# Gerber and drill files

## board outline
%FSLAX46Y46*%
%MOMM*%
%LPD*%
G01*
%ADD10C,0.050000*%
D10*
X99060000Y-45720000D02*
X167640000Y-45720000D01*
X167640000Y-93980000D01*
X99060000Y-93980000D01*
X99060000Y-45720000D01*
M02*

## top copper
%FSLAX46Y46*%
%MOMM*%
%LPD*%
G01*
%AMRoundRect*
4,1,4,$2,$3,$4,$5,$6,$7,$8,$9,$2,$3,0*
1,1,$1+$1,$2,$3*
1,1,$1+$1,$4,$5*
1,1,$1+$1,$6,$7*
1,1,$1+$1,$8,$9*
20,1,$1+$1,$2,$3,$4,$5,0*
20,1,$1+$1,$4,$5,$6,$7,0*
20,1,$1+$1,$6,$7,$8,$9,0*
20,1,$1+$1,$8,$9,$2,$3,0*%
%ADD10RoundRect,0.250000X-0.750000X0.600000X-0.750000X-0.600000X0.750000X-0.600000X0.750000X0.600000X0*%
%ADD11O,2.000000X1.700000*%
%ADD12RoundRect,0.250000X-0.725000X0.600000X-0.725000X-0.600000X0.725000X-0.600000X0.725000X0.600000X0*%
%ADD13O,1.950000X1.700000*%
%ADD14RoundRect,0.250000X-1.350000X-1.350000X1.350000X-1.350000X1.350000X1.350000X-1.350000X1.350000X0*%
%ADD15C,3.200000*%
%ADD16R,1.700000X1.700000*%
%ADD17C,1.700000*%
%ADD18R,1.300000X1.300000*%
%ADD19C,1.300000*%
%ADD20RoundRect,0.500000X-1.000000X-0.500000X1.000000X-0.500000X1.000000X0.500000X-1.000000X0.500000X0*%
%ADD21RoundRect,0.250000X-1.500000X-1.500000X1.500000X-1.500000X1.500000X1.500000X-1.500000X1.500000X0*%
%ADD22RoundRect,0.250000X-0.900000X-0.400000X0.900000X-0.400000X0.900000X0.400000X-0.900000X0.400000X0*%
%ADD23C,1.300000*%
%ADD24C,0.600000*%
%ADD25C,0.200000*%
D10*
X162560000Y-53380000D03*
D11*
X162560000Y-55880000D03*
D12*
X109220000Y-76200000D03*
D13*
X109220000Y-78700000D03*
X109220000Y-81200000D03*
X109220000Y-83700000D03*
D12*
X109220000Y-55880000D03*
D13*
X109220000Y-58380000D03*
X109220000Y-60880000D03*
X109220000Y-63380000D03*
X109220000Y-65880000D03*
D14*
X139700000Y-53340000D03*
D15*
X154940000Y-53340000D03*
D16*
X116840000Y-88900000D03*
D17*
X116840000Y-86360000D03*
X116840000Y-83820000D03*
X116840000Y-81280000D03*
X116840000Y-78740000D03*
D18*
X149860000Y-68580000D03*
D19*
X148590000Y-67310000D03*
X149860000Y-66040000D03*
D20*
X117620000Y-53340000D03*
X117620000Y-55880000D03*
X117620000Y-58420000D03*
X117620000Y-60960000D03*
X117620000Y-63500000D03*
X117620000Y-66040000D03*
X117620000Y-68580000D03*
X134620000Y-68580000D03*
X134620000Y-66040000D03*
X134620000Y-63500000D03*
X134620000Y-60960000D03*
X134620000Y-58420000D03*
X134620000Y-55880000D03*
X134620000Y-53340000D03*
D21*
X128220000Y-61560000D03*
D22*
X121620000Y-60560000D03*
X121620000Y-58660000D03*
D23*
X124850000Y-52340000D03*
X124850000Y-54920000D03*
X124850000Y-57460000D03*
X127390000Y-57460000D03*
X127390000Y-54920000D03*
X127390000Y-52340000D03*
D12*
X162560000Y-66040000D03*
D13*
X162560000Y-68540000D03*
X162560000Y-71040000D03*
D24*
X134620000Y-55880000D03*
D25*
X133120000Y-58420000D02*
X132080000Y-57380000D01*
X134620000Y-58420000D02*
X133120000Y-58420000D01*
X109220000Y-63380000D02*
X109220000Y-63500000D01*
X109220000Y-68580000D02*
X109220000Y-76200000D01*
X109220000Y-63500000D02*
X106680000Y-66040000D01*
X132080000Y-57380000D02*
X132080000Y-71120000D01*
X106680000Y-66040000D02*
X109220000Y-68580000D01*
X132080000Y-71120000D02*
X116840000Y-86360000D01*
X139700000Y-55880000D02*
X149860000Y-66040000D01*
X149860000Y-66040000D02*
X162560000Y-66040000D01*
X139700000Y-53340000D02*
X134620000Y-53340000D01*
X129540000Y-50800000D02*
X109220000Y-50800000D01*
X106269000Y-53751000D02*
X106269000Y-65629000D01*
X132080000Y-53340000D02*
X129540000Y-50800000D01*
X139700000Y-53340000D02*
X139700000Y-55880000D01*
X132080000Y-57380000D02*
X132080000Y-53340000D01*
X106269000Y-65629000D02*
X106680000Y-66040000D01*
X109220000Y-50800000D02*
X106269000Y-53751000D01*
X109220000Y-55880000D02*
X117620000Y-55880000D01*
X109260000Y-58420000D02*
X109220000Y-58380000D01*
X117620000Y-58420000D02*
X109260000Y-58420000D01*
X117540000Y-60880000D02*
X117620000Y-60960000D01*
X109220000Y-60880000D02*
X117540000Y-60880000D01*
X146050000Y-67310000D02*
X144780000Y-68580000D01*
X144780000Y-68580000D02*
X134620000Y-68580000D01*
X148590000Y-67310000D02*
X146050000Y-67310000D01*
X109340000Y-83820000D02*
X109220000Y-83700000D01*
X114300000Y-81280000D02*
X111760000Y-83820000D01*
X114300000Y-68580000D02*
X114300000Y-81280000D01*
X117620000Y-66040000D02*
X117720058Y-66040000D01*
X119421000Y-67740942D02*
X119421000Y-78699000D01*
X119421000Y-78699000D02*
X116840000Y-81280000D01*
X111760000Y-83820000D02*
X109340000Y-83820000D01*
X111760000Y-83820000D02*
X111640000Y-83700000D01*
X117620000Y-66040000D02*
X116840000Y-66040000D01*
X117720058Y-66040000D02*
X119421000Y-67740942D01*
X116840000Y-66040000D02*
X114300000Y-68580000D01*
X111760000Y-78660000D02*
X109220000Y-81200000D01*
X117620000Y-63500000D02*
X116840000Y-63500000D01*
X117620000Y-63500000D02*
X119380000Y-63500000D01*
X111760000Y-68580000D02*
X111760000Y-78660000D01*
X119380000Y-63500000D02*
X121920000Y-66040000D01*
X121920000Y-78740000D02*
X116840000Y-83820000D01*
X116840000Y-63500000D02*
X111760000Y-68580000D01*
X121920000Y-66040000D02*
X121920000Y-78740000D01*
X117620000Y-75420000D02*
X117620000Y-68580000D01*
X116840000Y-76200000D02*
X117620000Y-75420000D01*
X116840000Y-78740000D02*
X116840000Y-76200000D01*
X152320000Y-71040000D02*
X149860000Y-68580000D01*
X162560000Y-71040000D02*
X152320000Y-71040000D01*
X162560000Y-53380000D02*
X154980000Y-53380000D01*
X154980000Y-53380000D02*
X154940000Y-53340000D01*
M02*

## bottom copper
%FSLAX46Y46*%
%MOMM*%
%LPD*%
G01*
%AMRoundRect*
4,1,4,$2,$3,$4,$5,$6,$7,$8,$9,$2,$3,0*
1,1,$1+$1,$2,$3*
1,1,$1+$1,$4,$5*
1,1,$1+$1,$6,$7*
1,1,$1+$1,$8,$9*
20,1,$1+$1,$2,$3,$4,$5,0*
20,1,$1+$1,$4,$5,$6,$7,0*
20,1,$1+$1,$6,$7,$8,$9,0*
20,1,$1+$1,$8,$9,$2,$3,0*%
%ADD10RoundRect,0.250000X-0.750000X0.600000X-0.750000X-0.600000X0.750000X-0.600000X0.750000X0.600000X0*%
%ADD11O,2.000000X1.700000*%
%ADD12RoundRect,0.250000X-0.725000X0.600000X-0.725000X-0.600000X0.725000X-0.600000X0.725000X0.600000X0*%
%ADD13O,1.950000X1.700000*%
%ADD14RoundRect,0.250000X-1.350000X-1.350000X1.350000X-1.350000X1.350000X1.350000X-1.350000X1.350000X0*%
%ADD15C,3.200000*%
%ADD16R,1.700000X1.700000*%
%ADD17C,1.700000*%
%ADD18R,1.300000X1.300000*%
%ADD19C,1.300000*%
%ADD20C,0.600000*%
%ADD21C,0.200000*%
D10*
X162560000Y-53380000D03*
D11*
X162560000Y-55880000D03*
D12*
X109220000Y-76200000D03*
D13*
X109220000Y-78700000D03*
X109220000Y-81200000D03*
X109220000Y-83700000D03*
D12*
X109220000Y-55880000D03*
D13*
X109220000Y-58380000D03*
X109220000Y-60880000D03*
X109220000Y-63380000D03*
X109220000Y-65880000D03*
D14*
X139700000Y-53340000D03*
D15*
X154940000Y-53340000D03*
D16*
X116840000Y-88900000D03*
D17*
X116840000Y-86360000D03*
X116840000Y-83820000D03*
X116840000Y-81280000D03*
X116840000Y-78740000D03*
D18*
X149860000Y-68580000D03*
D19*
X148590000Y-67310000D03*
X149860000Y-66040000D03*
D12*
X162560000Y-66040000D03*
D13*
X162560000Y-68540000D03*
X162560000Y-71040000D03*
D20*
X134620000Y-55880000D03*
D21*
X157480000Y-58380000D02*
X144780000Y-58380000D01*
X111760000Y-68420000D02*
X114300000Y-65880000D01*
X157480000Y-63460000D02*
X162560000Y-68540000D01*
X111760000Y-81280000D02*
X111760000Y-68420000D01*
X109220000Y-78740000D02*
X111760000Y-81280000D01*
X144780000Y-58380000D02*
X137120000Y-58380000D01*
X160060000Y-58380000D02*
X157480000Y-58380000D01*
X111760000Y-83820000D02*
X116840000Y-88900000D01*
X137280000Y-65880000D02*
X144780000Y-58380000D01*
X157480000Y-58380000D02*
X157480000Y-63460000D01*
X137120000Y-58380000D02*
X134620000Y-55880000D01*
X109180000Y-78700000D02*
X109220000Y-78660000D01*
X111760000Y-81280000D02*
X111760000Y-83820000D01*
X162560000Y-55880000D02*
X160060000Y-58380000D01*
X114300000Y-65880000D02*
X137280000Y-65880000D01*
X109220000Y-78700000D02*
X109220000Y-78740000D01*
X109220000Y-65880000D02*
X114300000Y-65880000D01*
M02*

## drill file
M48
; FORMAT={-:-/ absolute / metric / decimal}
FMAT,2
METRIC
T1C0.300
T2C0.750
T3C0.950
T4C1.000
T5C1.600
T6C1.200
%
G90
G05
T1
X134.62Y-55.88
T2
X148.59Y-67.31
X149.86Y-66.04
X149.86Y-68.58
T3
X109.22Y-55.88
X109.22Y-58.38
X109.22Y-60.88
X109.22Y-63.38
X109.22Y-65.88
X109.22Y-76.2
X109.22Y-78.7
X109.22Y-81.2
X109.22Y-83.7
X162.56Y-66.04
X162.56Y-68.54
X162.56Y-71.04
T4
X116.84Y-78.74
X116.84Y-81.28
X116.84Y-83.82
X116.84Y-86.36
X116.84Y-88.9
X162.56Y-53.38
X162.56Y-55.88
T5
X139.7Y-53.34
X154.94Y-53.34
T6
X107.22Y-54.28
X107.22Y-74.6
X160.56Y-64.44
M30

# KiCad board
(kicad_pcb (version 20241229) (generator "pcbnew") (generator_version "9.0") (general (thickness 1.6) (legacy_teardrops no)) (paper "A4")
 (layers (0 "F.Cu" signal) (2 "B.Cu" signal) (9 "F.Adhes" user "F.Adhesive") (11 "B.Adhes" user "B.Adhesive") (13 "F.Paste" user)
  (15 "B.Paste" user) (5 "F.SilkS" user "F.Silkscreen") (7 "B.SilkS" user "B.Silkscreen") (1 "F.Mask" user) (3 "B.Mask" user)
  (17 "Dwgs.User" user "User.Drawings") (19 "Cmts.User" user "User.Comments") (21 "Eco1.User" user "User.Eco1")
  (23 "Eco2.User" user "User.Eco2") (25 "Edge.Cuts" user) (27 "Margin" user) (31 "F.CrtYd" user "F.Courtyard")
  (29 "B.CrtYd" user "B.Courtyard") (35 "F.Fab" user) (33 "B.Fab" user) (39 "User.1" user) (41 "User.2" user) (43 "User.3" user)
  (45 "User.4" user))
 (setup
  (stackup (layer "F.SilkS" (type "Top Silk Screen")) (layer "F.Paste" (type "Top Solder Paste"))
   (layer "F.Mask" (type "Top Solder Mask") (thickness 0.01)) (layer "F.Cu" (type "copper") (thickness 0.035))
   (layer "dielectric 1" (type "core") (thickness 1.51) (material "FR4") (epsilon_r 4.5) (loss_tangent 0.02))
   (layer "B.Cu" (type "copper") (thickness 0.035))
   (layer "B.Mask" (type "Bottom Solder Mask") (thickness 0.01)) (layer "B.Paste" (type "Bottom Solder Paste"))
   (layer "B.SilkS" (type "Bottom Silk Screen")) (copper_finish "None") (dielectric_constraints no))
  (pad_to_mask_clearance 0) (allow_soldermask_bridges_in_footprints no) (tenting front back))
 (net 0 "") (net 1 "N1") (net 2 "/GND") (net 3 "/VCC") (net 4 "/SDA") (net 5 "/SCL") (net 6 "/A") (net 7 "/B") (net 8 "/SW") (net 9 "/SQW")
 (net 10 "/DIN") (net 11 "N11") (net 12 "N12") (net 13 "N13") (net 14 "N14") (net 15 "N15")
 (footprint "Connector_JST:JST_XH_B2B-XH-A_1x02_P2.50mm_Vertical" (layer "F.Cu") (at 162.56 53.38 -90)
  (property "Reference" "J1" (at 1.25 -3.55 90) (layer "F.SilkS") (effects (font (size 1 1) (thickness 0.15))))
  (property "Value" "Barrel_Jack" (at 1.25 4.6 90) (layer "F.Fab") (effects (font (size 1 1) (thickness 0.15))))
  (pad "1" thru_hole roundrect (at 0 0 270) (size 1.7 2) (drill 1) (layers "*.Cu" "*.Mask") (remove_unused_layers no)
   (roundrect_rratio 0.147059) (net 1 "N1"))
  (pad "2" thru_hole oval (at 2.5 0 270) (size 1.7 2) (drill 1) (layers "*.Cu" "*.Mask") (remove_unused_layers no) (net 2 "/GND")))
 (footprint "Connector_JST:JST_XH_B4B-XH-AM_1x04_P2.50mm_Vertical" (layer "F.Cu") (at 109.22 76.2 -90)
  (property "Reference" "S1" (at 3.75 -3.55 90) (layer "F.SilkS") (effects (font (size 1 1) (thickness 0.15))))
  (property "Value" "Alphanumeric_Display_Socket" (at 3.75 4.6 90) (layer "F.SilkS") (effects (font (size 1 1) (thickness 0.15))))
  (pad "" np_thru_hole circle (at -1.6 2 270) (size 1.2 1.2) (drill 1.2) (layers "*.Cu" "*.Mask"))
  (pad "1" thru_hole roundrect (at 0 0 270) (size 1.7 1.95) (drill 0.95) (layers "*.Cu" "*.Mask") (remove_unused_layers no)
   (roundrect_rratio 0.147059) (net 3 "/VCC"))
  (pad "2" thru_hole oval (at 2.5 0 270) (size 1.7 1.95) (drill 0.95) (layers "*.Cu" "*.Mask") (remove_unused_layers no) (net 2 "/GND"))
  (pad "3" thru_hole oval (at 5 0 270) (size 1.7 1.95) (drill 0.95) (layers "*.Cu" "*.Mask") (remove_unused_layers no) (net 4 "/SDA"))
  (pad "4" thru_hole oval (at 7.5 0 270) (size 1.7 1.95) (drill 0.95) (layers "*.Cu" "*.Mask") (remove_unused_layers no) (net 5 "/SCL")))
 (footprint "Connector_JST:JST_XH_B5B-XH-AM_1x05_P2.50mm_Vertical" (layer "F.Cu") (at 109.22 55.88 -90)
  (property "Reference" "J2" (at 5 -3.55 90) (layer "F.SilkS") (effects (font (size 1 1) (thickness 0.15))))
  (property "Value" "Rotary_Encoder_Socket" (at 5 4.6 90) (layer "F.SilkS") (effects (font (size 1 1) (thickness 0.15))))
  (pad "" np_thru_hole circle (at -1.6 2 270) (size 1.2 1.2) (drill 1.2) (layers "*.Cu" "*.Mask"))
  (pad "1" thru_hole roundrect (at 0 0 270) (size 1.7 1.95) (drill 0.95) (layers "*.Cu" "*.Mask") (remove_unused_layers no)
   (roundrect_rratio 0.147059) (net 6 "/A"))
  (pad "2" thru_hole oval (at 2.5 0 270) (size 1.7 1.95) (drill 0.95) (layers "*.Cu" "*.Mask") (remove_unused_layers no) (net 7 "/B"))
  (pad "3" thru_hole oval (at 5 0 270) (size 1.7 1.95) (drill 0.95) (layers "*.Cu" "*.Mask") (remove_unused_layers no) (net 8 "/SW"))
  (pad "4" thru_hole oval (at 7.5 0 270) (size 1.7 1.95) (drill 0.95) (layers "*.Cu" "*.Mask") (remove_unused_layers no) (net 3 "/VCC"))
  (pad "5" thru_hole oval (at 10 0 270) (size 1.7 1.95) (drill 0.95) (layers "*.Cu" "*.Mask") (remove_unused_layers no) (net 2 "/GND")))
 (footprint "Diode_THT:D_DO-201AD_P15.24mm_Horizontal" (layer "F.Cu") (at 139.7 53.34)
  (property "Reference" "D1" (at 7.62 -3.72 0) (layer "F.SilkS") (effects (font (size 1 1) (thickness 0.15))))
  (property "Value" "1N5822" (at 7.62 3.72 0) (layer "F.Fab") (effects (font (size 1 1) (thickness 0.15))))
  (pad "1" thru_hole roundrect (at 0 0) (size 3.2 3.2) (drill 1.6) (layers "*.Cu" "*.Mask") (remove_unused_layers no)
   (roundrect_rratio 0.078125) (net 3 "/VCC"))
  (pad "2" thru_hole circle (at 15.24 0) (size 3.2 3.2) (drill 1.6) (layers "*.Cu" "*.Mask") (remove_unused_layers no) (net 1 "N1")))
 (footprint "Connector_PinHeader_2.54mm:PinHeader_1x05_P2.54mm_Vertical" (layer "F.Cu") (at 116.84 88.9 180)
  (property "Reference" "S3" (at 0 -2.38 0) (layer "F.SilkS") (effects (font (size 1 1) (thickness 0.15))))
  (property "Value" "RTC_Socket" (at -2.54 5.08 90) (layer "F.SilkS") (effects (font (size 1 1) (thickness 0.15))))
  (pad "1" thru_hole rect (at 0 0 180) (size 1.7 1.7) (drill 1) (layers "*.Cu" "*.Mask") (remove_unused_layers no) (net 2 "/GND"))
  (pad "2" thru_hole circle (at 0 2.54 180) (size 1.7 1.7) (drill 1) (layers "*.Cu" "*.Mask") (remove_unused_layers no) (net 3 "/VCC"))
  (pad "3" thru_hole circle (at 0 5.08 180) (size 1.7 1.7) (drill 1) (layers "*.Cu" "*.Mask") (remove_unused_layers no) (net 4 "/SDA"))
  (pad "4" thru_hole circle (at 0 7.62 180) (size 1.7 1.7) (drill 1) (layers "*.Cu" "*.Mask") (remove_unused_layers no) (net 5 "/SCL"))
  (pad "5" thru_hole circle (at 0 10.16 180) (size 1.7 1.7) (drill 1) (layers "*.Cu" "*.Mask") (remove_unused_layers no) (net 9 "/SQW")))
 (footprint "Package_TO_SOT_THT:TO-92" (layer "F.Cu") (at 149.86 68.58 90)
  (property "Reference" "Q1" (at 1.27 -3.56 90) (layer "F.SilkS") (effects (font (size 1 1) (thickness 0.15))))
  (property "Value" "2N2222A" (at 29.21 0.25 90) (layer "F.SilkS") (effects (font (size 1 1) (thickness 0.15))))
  (pad "1" thru_hole rect (at 0 0 90) (size 1.3 1.3) (drill 0.75) (layers "*.Cu" "*.Mask") (remove_unused_layers no) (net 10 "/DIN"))
  (pad "2" thru_hole circle (at 1.27 -1.27 90) (size 1.3 1.3) (drill 0.75) (layers "*.Cu" "*.Mask") (remove_unused_layers no) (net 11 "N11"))
  (pad "3" thru_hole circle (at 2.54 0 90) (size 1.3 1.3) (drill 0.75) (layers "*.Cu" "*.Mask") (remove_unused_layers no) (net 3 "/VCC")))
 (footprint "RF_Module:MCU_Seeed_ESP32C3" (layer "F.Cu") (at 126.12 60.96)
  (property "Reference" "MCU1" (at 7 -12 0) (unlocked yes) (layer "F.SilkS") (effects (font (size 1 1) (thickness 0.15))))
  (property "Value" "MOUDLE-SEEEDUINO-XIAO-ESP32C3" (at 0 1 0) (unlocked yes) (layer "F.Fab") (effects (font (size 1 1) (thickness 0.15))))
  (pad "" smd roundrect (at 1.1 -0.4) (size 1.5 1.5) (layers "F.Paste") (roundrect_rratio 0.1666666667))
  (pad "" smd roundrect (at 1.1 1.6) (size 1.5 1.5) (layers "F.Paste") (roundrect_rratio 0.1666666667))
  (pad "" smd roundrect (at 3.1 -0.4) (size 1.5 1.5) (layers "F.Paste") (roundrect_rratio 0.1666666667))
  (pad "" smd roundrect (at 3.1 1.6) (size 1.5 1.5) (layers "F.Paste") (roundrect_rratio 0.1666666667))
  (pad "1" smd roundrect (at -8.5 -7.62) (size 3 2) (layers "F.Cu" "F.Mask" "F.Paste") (roundrect_rratio 0.25) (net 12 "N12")
   (thermal_bridge_angle 45))
  (pad "2" smd roundrect (at -8.5 -5.08) (size 3 2) (layers "F.Cu" "F.Mask" "F.Paste") (roundrect_rratio 0.25) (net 6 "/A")
   (thermal_bridge_angle 45))
  (pad "3" smd roundrect (at -8.5 -2.54) (size 3 2) (layers "F.Cu" "F.Mask" "F.Paste") (roundrect_rratio 0.25) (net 7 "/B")
   (thermal_bridge_angle 45))
  (pad "4" smd roundrect (at -8.5 0) (size 3 2) (layers "F.Cu" "F.Mask" "F.Paste") (roundrect_rratio 0.25) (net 8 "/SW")
   (thermal_bridge_angle 45))
  (pad "5" smd roundrect (at -8.5 2.54) (size 3 2) (layers "F.Cu" "F.Mask" "F.Paste") (roundrect_rratio 0.25) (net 4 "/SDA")
   (thermal_bridge_angle 45))
  (pad "6" smd roundrect (at -8.5 5.08) (size 3 2) (layers "F.Cu" "F.Mask" "F.Paste") (roundrect_rratio 0.25) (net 5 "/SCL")
   (thermal_bridge_angle 45))
  (pad "7" smd roundrect (at -8.5 7.62) (size 3 2) (layers "F.Cu" "F.Mask" "F.Paste") (roundrect_rratio 0.25) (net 9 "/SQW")
   (thermal_bridge_angle 45))
  (pad "8" smd roundrect (at 8.5 7.62) (size 3 2) (layers "F.Cu" "F.Mask" "F.Paste") (roundrect_rratio 0.25) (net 11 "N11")
   (thermal_bridge_angle 45))
  (pad "9" smd roundrect (at 8.5 5.08) (size 3 2) (layers "F.Cu" "F.Mask" "F.Paste") (roundrect_rratio 0.25) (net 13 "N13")
   (thermal_bridge_angle 45))
  (pad "10" smd roundrect (at 8.5 2.54) (size 3 2) (layers "F.Cu" "F.Mask" "F.Paste") (roundrect_rratio 0.25) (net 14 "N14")
   (thermal_bridge_angle 45))
  (pad "11" smd roundrect (at 8.5 0) (size 3 2) (layers "F.Cu" "F.Mask" "F.Paste") (roundrect_rratio 0.25) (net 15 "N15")
   (thermal_bridge_angle 45))
  (pad "12" smd roundrect (at 8.5 -2.54) (size 3 2) (layers "F.Cu" "F.Mask" "F.Paste") (roundrect_rratio 0.25) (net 3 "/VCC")
   (thermal_bridge_angle 45))
  (pad "13" smd roundrect (at 8.5 -5.08) (size 3 2) (layers "F.Cu" "F.Mask" "F.Paste") (roundrect_rratio 0.25) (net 2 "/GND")
   (thermal_bridge_angle 45))
  (pad "14" smd roundrect (at 8.5 -7.62) (size 3 2) (layers "F.Cu" "F.Mask" "F.Paste") (roundrect_rratio 0.25) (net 3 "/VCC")
   (thermal_bridge_angle 45))
  (pad "15" smd roundrect (at 2.1 0.6) (size 3.5 3.5) (layers "F.Cu" "F.Mask") (roundrect_rratio 0.07142857143))
  (pad "16" smd roundrect (at -4.5 -0.4) (size 2.3 1.3) (layers "F.Cu" "F.Mask" "F.Paste") (roundrect_rratio 0.1923076923))
  (pad "17" smd roundrect (at -4.5 -2.3) (size 2.3 1.3) (layers "F.Cu" "F.Mask" "F.Paste") (roundrect_rratio 0.1923076923))
  (pad "18" smd circle (at -1.27 -8.62) (size 1.3 1.3) (layers "F.Cu" "F.Mask" "F.Paste"))
  (pad "19" smd circle (at -1.27 -6.04) (size 1.3 1.3) (layers "F.Cu" "F.Mask" "F.Paste"))
  (pad "20" smd circle (at -1.27 -3.5) (size 1.3 1.3) (layers "F.Cu" "F.Mask" "F.Paste"))
  (pad "21" smd circle (at 1.27 -3.5) (size 1.3 1.3) (layers "F.Cu" "F.Mask" "F.Paste"))
  (pad "22" smd circle (at 1.27 -6.04) (size 1.3 1.3) (layers "F.Cu" "F.Mask" "F.Paste"))
  (pad "23" smd circle (at 1.27 -8.62) (size 1.3 1.3) (layers "F.Cu" "F.Mask" "F.Paste")))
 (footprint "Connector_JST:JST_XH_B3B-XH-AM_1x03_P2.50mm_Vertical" (layer "F.Cu") (at 162.56 66.04 -90)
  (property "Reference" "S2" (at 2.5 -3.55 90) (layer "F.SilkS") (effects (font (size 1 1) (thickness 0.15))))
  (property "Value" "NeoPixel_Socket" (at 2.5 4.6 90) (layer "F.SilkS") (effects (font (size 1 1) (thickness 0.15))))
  (pad "" np_thru_hole circle (at -1.6 2 270) (size 1.2 1.2) (drill 1.2) (layers "*.Cu" "*.Mask"))
  (pad "1" thru_hole roundrect (at 0 0 270) (size 1.7 1.95) (drill 0.95) (layers "*.Cu" "*.Mask") (remove_unused_layers no)
   (roundrect_rratio 0.147059) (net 3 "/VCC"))
  (pad "2" thru_hole oval (at 2.5 0 270) (size 1.7 1.95) (drill 0.95) (layers "*.Cu" "*.Mask") (remove_unused_layers no) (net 2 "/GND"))
  (pad "3" thru_hole oval (at 5 0 270) (size 1.7 1.95) (drill 0.95) (layers "*.Cu" "*.Mask") (remove_unused_layers no) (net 10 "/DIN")))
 (gr_rect (start 99.06 45.72) (end 167.64 93.98) (stroke (width 0.05) (type default)) (fill no) (layer "Edge.Cuts"))
 (via (at 134.62 55.88) (size 0.6) (drill 0.3) (layers "F.Cu" "B.Cu") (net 2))
 (segment (start 157.48 58.38) (end 144.78 58.38) (width 0.2) (layer "B.Cu") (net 2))
 (segment (start 111.76 68.42) (end 114.3 65.88) (width 0.2) (layer "B.Cu") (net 2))
 (segment (start 157.48 63.46) (end 162.56 68.54) (width 0.2) (layer "B.Cu") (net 2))
 (segment (start 111.76 81.28) (end 111.76 68.42) (width 0.2) (layer "B.Cu") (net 2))
 (segment (start 109.22 78.74) (end 111.76 81.28) (width 0.2) (layer "B.Cu") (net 2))
 (segment (start 144.78 58.38) (end 137.12 58.38) (width 0.2) (layer "B.Cu") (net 2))
 (segment (start 160.06 58.38) (end 157.48 58.38) (width 0.2) (layer "B.Cu") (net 2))
 (segment (start 111.76 83.82) (end 116.84 88.9) (width 0.2) (layer "B.Cu") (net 2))
 (segment (start 137.28 65.88) (end 144.78 58.38) (width 0.2) (layer "B.Cu") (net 2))
 (segment (start 157.48 58.38) (end 157.48 63.46) (width 0.2) (layer "B.Cu") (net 2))
 (segment (start 137.12 58.38) (end 134.62 55.88) (width 0.2) (layer "B.Cu") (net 2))
 (segment (start 109.18 78.7) (end 109.22 78.66) (width 0.2) (layer "B.Cu") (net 2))
 (segment (start 111.76 81.28) (end 111.76 83.82) (width 0.2) (layer "B.Cu") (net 2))
 (segment (start 162.56 55.88) (end 160.06 58.38) (width 0.2) (layer "B.Cu") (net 2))
 (segment (start 114.3 65.88) (end 137.28 65.88) (width 0.2) (layer "B.Cu") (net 2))
 (segment (start 109.22 78.7) (end 109.22 78.74) (width 0.2) (layer "B.Cu") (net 2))
 (segment (start 109.22 65.88) (end 114.3 65.88) (width 0.2) (layer "B.Cu") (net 2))
 (segment (start 133.12 58.42) (end 132.08 57.38) (width 0.2) (layer "F.Cu") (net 3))
 (segment (start 134.62 58.42) (end 133.12 58.42) (width 0.2) (layer "F.Cu") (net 3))
 (segment (start 109.22 63.38) (end 109.22 63.5) (width 0.2) (layer "F.Cu") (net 3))
 (segment (start 109.22 68.58) (end 109.22 76.2) (width 0.2) (layer "F.Cu") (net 3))
 (segment (start 109.22 63.5) (end 106.68 66.04) (width 0.2) (layer "F.Cu") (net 3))
 (segment (start 132.08 57.38) (end 132.08 71.12) (width 0.2) (layer "F.Cu") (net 3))
 (segment (start 106.68 66.04) (end 109.22 68.58) (width 0.2) (layer "F.Cu") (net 3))
 (segment (start 132.08 71.12) (end 116.84 86.36) (width 0.2) (layer "F.Cu") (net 3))
 (segment (start 139.7 55.88) (end 149.86 66.04) (width 0.2) (layer "F.Cu") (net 3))
 (segment (start 149.86 66.04) (end 162.56 66.04) (width 0.2) (layer "F.Cu") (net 3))
 (segment (start 139.7 53.34) (end 134.62 53.34) (width 0.2) (layer "F.Cu") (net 3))
 (segment (start 129.54 50.8) (end 109.22 50.8) (width 0.2) (layer "F.Cu") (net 3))
 (segment (start 106.269 53.751) (end 106.269 65.629) (width 0.2) (layer "F.Cu") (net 3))
 (segment (start 132.08 53.34) (end 129.54 50.8) (width 0.2) (layer "F.Cu") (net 3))
 (segment (start 139.7 53.34) (end 139.7 55.88) (width 0.2) (layer "F.Cu") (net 3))
 (segment (start 132.08 57.38) (end 132.08 53.34) (width 0.2) (layer "F.Cu") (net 3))
 (segment (start 106.269 65.629) (end 106.68 66.04) (width 0.2) (layer "F.Cu") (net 3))
 (segment (start 109.22 50.8) (end 106.269 53.751) (width 0.2) (layer "F.Cu") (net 3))
 (segment (start 109.22 55.88) (end 117.62 55.88) (width 0.2) (layer "F.Cu") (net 6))
 (segment (start 109.26 58.42) (end 109.22 58.38) (width 0.2) (layer "F.Cu") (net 7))
 (segment (start 117.62 58.42) (end 109.26 58.42) (width 0.2) (layer "F.Cu") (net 7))
 (segment (start 117.54 60.88) (end 117.62 60.96) (width 0.2) (layer "F.Cu") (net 8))
 (segment (start 109.22 60.88) (end 117.54 60.88) (width 0.2) (layer "F.Cu") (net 8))
 (segment (start 146.05 67.31) (end 144.78 68.58) (width 0.2) (layer "F.Cu") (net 11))
 (segment (start 144.78 68.58) (end 134.62 68.58) (width 0.2) (layer "F.Cu") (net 11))
 (segment (start 148.59 67.31) (end 146.05 67.31) (width 0.2) (layer "F.Cu") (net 11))
 (segment (start 109.34 83.82) (end 109.22 83.7) (width 0.2) (layer "F.Cu") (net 5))
 (segment (start 114.3 81.28) (end 111.76 83.82) (width 0.2) (layer "F.Cu") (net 5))
 (segment (start 114.3 68.58) (end 114.3 81.28) (width 0.2) (layer "F.Cu") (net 5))
 (segment (start 117.62 66.04) (end 117.720058 66.04) (width 0.2) (layer "F.Cu") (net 5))
 (segment (start 119.421 67.740942) (end 119.421 78.699) (width 0.2) (layer "F.Cu") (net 5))
 (segment (start 119.421 78.699) (end 116.84 81.28) (width 0.2) (layer "F.Cu") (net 5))
 (segment (start 111.76 83.82) (end 109.34 83.82) (width 0.2) (layer "F.Cu") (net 5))
 (segment (start 111.76 83.82) (end 111.64 83.7) (width 0.2) (layer "F.Cu") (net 5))
 (segment (start 117.62 66.04) (end 116.84 66.04) (width 0.2) (layer "F.Cu") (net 5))
 (segment (start 117.720058 66.04) (end 119.421 67.740942) (width 0.2) (layer "F.Cu") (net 5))
 (segment (start 116.84 66.04) (end 114.3 68.58) (width 0.2) (layer "F.Cu") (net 5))
 (segment (start 111.76 78.66) (end 109.22 81.2) (width 0.2) (layer "F.Cu") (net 4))
 (segment (start 117.62 63.5) (end 116.84 63.5) (width 0.2) (layer "F.Cu") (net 4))
 (segment (start 117.62 63.5) (end 119.38 63.5) (width 0.2) (layer "F.Cu") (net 4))
 (segment (start 111.76 68.58) (end 111.76 78.66) (width 0.2) (layer "F.Cu") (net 4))
 (segment (start 119.38 63.5) (end 121.92 66.04) (width 0.2) (layer "F.Cu") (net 4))
 (segment (start 121.92 78.74) (end 116.84 83.82) (width 0.2) (layer "F.Cu") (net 4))
 (segment (start 116.84 63.5) (end 111.76 68.58) (width 0.2) (layer "F.Cu") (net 4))
 (segment (start 121.92 66.04) (end 121.92 78.74) (width 0.2) (layer "F.Cu") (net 4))
 (segment (start 117.62 75.42) (end 117.62 68.58) (width 0.2) (layer "F.Cu") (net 9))
 (segment (start 116.84 76.2) (end 117.62 75.42) (width 0.2) (layer "F.Cu") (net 9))
 (segment (start 116.84 78.74) (end 116.84 76.2) (width 0.2) (layer "F.Cu") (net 9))
 (segment (start 152.32 71.04) (end 149.86 68.58) (width 0.2) (layer "F.Cu") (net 10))
 (segment (start 162.56 71.04) (end 152.32 71.04) (width 0.2) (layer "F.Cu") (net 10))
 (segment (start 162.56 53.38) (end 154.98 53.38) (width 0.2) (layer "F.Cu") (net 1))
 (segment (start 154.98 53.38) (end 154.94 53.34) (width 0.2) (layer "F.Cu") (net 1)))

